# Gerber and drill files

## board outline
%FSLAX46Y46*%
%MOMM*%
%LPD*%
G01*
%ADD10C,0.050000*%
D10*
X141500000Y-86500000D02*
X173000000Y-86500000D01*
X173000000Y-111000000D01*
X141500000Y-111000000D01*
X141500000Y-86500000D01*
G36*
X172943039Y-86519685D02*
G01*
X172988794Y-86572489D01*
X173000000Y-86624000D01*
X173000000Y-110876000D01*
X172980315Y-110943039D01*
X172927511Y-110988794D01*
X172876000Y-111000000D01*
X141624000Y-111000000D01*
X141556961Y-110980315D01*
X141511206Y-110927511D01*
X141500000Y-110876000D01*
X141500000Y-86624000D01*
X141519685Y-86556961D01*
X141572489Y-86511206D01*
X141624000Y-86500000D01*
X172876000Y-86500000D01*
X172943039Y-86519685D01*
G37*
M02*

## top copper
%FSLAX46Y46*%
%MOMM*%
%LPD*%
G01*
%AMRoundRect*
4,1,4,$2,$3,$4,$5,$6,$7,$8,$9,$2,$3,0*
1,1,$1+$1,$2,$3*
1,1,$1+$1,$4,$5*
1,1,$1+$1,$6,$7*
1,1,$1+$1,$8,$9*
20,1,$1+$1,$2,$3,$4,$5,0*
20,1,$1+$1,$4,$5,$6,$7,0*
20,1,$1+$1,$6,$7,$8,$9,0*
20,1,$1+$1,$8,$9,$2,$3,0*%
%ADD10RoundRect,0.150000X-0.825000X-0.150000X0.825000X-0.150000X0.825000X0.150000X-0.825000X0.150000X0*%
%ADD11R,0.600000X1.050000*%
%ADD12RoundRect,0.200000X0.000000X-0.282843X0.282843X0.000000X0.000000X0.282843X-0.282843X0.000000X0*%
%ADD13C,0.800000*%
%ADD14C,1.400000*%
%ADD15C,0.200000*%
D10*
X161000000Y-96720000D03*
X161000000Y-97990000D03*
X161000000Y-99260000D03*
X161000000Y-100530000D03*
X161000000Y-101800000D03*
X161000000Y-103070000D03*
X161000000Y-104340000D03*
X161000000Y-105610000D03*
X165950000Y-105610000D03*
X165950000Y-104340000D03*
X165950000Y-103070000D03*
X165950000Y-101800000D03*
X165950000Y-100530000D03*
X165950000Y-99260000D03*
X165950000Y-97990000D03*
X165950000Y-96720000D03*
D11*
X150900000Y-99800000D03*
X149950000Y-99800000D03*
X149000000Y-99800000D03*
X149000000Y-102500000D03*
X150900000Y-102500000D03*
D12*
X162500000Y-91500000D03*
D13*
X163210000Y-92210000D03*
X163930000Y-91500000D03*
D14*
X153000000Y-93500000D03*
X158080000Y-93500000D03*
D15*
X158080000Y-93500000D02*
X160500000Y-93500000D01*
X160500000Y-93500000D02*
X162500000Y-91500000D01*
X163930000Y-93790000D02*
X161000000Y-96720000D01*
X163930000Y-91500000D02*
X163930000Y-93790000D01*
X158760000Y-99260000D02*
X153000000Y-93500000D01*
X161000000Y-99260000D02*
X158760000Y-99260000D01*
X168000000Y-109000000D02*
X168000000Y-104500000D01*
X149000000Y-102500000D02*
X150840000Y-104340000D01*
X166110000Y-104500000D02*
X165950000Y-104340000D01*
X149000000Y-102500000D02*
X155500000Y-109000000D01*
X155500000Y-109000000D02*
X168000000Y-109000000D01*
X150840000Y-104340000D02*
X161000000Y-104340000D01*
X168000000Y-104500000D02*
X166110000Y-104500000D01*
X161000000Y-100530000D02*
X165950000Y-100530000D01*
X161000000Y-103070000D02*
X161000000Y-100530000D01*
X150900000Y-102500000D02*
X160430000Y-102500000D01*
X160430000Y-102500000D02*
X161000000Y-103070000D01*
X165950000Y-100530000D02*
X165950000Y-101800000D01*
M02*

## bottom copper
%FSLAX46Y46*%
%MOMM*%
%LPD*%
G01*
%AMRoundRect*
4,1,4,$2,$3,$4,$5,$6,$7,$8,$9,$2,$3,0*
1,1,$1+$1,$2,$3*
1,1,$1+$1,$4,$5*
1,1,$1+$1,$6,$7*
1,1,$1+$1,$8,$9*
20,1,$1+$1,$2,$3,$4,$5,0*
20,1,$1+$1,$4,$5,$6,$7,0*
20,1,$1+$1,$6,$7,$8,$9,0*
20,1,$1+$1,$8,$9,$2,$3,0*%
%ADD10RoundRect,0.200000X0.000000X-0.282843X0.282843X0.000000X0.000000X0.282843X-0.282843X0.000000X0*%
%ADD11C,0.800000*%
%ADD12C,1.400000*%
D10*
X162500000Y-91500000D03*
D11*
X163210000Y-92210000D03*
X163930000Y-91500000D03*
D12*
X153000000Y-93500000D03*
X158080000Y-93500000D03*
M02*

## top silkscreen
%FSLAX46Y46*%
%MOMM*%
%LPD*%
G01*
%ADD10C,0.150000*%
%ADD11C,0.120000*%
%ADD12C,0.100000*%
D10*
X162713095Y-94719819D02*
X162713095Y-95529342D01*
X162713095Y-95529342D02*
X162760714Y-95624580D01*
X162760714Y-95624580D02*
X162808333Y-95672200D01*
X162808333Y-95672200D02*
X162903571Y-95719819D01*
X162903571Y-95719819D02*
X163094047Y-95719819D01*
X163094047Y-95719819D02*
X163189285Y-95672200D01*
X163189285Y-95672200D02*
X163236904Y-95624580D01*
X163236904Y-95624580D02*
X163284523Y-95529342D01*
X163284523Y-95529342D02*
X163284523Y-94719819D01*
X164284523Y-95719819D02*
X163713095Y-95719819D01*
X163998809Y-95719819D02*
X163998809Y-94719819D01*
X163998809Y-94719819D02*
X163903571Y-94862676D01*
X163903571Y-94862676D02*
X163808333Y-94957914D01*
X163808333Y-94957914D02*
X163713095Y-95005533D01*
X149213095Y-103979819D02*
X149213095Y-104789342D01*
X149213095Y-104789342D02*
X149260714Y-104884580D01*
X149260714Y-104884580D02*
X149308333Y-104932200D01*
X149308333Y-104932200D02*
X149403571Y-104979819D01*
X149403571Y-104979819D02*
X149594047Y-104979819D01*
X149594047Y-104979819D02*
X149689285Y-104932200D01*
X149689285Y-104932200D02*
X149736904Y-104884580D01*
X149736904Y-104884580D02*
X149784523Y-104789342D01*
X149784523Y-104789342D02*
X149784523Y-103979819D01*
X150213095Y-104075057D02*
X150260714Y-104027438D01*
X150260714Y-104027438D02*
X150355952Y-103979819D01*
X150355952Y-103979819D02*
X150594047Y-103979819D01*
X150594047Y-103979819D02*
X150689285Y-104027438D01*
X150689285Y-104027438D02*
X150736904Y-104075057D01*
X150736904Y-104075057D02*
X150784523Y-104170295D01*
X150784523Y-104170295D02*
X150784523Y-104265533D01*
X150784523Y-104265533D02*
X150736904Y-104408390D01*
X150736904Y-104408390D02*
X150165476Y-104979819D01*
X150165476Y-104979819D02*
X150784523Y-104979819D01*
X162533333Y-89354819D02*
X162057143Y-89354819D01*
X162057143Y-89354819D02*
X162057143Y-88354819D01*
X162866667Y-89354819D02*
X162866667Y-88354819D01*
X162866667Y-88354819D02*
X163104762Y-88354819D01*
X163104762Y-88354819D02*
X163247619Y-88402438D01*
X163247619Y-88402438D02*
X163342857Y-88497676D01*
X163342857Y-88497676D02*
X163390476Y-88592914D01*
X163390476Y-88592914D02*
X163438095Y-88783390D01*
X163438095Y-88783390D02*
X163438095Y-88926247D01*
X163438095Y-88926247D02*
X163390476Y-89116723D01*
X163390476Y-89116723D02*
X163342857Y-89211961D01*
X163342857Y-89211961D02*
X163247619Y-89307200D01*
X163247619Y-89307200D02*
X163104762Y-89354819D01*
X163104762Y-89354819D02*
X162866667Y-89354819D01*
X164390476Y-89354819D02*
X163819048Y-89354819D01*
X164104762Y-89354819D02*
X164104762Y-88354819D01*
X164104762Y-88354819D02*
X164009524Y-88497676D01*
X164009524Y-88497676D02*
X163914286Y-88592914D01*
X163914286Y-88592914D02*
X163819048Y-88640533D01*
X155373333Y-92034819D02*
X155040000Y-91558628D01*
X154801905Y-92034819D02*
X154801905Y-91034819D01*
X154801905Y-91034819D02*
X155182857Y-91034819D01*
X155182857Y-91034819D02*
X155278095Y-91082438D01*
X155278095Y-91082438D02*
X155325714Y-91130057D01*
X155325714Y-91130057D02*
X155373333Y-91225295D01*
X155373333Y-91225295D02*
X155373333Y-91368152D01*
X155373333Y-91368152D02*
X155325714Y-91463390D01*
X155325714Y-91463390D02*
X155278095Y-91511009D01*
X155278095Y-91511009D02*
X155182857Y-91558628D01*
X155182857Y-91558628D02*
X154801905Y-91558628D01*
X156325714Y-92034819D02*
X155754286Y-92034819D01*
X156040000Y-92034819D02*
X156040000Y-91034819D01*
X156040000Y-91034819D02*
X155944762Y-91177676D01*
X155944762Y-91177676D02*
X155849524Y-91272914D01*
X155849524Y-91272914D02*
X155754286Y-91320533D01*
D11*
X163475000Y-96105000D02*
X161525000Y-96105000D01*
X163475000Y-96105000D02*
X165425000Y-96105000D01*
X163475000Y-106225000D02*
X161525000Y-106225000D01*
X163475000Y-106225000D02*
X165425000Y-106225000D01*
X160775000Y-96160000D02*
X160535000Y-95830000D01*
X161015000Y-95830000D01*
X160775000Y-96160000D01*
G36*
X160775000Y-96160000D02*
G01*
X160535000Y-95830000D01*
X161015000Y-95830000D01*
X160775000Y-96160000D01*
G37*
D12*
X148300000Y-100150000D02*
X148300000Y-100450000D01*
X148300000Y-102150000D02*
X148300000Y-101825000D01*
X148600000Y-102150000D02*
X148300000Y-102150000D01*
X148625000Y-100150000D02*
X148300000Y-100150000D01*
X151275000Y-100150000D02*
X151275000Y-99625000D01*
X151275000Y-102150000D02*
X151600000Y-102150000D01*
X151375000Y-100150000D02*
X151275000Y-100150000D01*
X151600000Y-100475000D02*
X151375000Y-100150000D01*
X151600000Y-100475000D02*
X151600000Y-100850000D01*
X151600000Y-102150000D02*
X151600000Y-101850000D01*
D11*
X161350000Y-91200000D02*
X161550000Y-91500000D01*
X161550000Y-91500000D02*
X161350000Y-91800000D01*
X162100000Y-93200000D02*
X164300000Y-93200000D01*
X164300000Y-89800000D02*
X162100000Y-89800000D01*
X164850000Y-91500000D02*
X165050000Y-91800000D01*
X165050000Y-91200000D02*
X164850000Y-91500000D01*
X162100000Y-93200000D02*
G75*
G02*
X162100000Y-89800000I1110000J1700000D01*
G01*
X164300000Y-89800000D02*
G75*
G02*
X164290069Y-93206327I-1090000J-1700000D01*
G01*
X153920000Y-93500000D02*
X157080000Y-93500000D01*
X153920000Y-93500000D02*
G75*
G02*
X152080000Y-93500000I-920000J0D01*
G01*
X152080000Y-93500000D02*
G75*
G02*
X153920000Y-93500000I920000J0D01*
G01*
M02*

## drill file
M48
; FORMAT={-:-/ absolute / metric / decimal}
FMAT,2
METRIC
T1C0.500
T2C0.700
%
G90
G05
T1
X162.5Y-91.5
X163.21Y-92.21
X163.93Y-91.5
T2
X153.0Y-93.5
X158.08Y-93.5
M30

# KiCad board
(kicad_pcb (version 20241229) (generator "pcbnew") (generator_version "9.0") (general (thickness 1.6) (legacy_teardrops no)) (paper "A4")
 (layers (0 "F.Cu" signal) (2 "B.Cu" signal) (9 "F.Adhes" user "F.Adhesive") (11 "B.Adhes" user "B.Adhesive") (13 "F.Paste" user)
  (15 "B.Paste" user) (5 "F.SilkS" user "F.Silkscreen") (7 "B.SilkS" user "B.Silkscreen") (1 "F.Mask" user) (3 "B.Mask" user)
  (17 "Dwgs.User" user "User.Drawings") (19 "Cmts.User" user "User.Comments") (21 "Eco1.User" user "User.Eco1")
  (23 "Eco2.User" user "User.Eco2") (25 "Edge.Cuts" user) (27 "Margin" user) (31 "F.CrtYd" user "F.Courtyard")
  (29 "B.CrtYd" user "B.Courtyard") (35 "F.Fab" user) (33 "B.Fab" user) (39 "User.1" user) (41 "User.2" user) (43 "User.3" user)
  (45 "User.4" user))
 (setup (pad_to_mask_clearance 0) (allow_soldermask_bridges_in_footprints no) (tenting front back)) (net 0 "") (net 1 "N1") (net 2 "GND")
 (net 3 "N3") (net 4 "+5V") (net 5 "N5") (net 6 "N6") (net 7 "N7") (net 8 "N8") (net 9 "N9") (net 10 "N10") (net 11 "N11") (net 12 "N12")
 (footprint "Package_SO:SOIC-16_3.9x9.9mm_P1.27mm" (layer "F.Cu") (at 163.475 101.165)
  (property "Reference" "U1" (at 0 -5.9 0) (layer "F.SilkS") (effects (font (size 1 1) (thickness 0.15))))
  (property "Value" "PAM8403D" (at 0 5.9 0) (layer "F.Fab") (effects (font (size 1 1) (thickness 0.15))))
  (fp_line (start 0 -5.06) (end -1.95 -5.06) (stroke (width 0.12) (type solid)) (layer "F.SilkS"))
  (fp_line (start 0 -5.06) (end 1.95 -5.06) (stroke (width 0.12) (type solid)) (layer "F.SilkS"))
  (fp_line (start 0 5.06) (end -1.95 5.06) (stroke (width 0.12) (type solid)) (layer "F.SilkS"))
  (fp_line (start 0 5.06) (end 1.95 5.06) (stroke (width 0.12) (type solid)) (layer "F.SilkS"))
  (fp_poly (pts (xy -2.7 -5.005) (xy -2.94 -5.335) (xy -2.46 -5.335)) (stroke (width 0.12) (type solid)) (fill yes) (layer "F.SilkS"))
  (pad "1" smd roundrect (at -2.475 -4.445) (size 1.95 0.6) (layers "F.Cu" "F.Mask" "F.Paste") (roundrect_rratio 0.25) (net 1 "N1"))
  (pad "2" smd roundrect (at -2.475 -3.175) (size 1.95 0.6) (layers "F.Cu" "F.Mask" "F.Paste") (roundrect_rratio 0.25) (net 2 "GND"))
  (pad "3" smd roundrect (at -2.475 -1.905) (size 1.95 0.6) (layers "F.Cu" "F.Mask" "F.Paste") (roundrect_rratio 0.25) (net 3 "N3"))
  (pad "4" smd roundrect (at -2.475 -0.635) (size 1.95 0.6) (layers "F.Cu" "F.Mask" "F.Paste") (roundrect_rratio 0.25) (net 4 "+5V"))
  (pad "5" smd roundrect (at -2.475 0.635) (size 1.95 0.6) (layers "F.Cu" "F.Mask" "F.Paste") (roundrect_rratio 0.25) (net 4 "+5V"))
  (pad "6" smd roundrect (at -2.475 1.905) (size 1.95 0.6) (layers "F.Cu" "F.Mask" "F.Paste") (roundrect_rratio 0.25) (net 4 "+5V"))
  (pad "7" smd roundrect (at -2.475 3.175) (size 1.95 0.6) (layers "F.Cu" "F.Mask" "F.Paste") (roundrect_rratio 0.25) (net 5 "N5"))
  (pad "8" smd roundrect (at -2.475 4.445) (size 1.95 0.6) (layers "F.Cu" "F.Mask" "F.Paste") (roundrect_rratio 0.25) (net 2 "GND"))
  (pad "9" smd roundrect (at 2.475 4.445) (size 1.95 0.6) (layers "F.Cu" "F.Mask" "F.Paste") (roundrect_rratio 0.25) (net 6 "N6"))
  (pad "10" smd roundrect (at 2.475 3.175) (size 1.95 0.6) (layers "F.Cu" "F.Mask" "F.Paste") (roundrect_rratio 0.25) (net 5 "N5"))
  (pad "11" smd roundrect (at 2.475 1.905) (size 1.95 0.6) (layers "F.Cu" "F.Mask" "F.Paste") (roundrect_rratio 0.25) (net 2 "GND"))
  (pad "12" smd roundrect (at 2.475 0.635) (size 1.95 0.6) (layers "F.Cu" "F.Mask" "F.Paste") (roundrect_rratio 0.25) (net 4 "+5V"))
  (pad "13" smd roundrect (at 2.475 -0.635) (size 1.95 0.6) (layers "F.Cu" "F.Mask" "F.Paste") (roundrect_rratio 0.25) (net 4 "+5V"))
  (pad "14" smd roundrect (at 2.475 -1.905) (size 1.95 0.6) (layers "F.Cu" "F.Mask" "F.Paste") (roundrect_rratio 0.25) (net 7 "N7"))
  (pad "15" smd roundrect (at 2.475 -3.175) (size 1.95 0.6) (layers "F.Cu" "F.Mask" "F.Paste") (roundrect_rratio 0.25) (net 2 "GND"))
  (pad "16" smd roundrect (at 2.475 -4.445) (size 1.95 0.6) (layers "F.Cu" "F.Mask" "F.Paste") (roundrect_rratio 0.25) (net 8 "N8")))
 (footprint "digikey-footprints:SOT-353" (layer "F.Cu") (at 149.95 101.15 180)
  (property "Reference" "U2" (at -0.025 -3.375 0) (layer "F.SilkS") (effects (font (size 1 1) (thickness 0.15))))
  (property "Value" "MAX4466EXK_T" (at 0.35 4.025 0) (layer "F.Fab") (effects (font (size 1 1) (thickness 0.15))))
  (fp_line (start 1.65 1) (end 1.65 0.7) (stroke (width 0.1) (type solid)) (layer "F.SilkS"))
  (fp_line (start 1.65 -1) (end 1.65 -0.675) (stroke (width 0.1) (type solid)) (layer "F.SilkS"))
  (fp_line (start 1.35 -1) (end 1.65 -1) (stroke (width 0.1) (type solid)) (layer "F.SilkS"))
  (fp_line (start 1.325 1) (end 1.65 1) (stroke (width 0.1) (type solid)) (layer "F.SilkS"))
  (fp_line (start -1.325 1) (end -1.325 1.525) (stroke (width 0.1) (type solid)) (layer "F.SilkS"))
  (fp_line (start -1.325 -1) (end -1.65 -1) (stroke (width 0.1) (type solid)) (layer "F.SilkS"))
  (fp_line (start -1.425 1) (end -1.325 1) (stroke (width 0.1) (type solid)) (layer "F.SilkS"))
  (fp_line (start -1.65 0.675) (end -1.425 1) (stroke (width 0.1) (type solid)) (layer "F.SilkS"))
  (fp_line (start -1.65 0.675) (end -1.65 0.3) (stroke (width 0.1) (type solid)) (layer "F.SilkS"))
  (fp_line (start -1.65 -1) (end -1.65 -0.7) (stroke (width 0.1) (type solid)) (layer "F.SilkS"))
  (pad "1" smd rect (at -0.95 1.35 180) (size 0.6 1.05) (layers "F.Cu" "F.Mask" "F.Paste") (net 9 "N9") (solder_mask_margin 0.07))
  (pad "2" smd rect (at 0 1.35 180) (size 0.6 1.05) (layers "F.Cu" "F.Mask" "F.Paste") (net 2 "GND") (solder_mask_margin 0.07))
  (pad "3" smd rect (at 0.95 1.35 180) (size 0.6 1.05) (layers "F.Cu" "F.Mask" "F.Paste") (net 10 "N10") (solder_mask_margin 0.07))
  (pad "4" smd rect (at 0.95 -1.35 180) (size 0.6 1.05) (layers "F.Cu" "F.Mask" "F.Paste") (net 5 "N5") (solder_mask_margin 0.07))
  (pad "5" smd rect (at -0.95 -1.35 180) (size 0.6 1.05) (layers "F.Cu" "F.Mask" "F.Paste") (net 4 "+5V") (solder_mask_margin 0.07)))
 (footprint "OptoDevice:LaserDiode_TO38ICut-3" (layer "F.Cu") (at 162.5 91.5)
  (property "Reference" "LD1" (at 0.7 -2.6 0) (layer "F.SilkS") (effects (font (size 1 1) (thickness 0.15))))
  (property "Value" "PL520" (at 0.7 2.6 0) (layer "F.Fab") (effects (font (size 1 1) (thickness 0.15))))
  (fp_line (start -1.15 -0.3) (end -0.95 0) (stroke (width 0.12) (type solid)) (layer "F.SilkS"))
  (fp_line (start -0.95 0) (end -1.15 0.3) (stroke (width 0.12) (type solid)) (layer "F.SilkS"))
  (fp_line (start -0.4 1.7) (end 1.8 1.7) (stroke (width 0.12) (type solid)) (layer "F.SilkS"))
  (fp_line (start 1.8 -1.7) (end -0.4 -1.7) (stroke (width 0.12) (type solid)) (layer "F.SilkS"))
  (fp_line (start 2.35 0) (end 2.55 0.3) (stroke (width 0.12) (type solid)) (layer "F.SilkS"))
  (fp_line (start 2.55 -0.3) (end 2.35 0) (stroke (width 0.12) (type solid)) (layer "F.SilkS"))
  (fp_arc (start -0.4 1.7) (mid -1.320296 0) (end -0.4 -1.7) (stroke (width 0.12) (type solid)) (layer "F.SilkS"))
  (fp_arc (start 1.8 -1.7) (mid 2.729422 0.005888) (end 1.790069 1.706327) (stroke (width 0.12) (type solid)) (layer "F.SilkS"))
  (pad "1" thru_hole roundrect (at 0 0 45) (size 0.8 0.8) (drill 0.5) (layers "*.Cu" "*.Mask") (remove_unused_layers no)
   (roundrect_rratio 0.25) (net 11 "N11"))
  (pad "2" thru_hole circle (at 0.71 0.71) (size 0.8 0.8) (drill 0.5) (layers "*.Cu" "*.Mask") (remove_unused_layers no) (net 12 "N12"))
  (pad "3" thru_hole circle (at 1.43 0) (size 0.8 0.8) (drill 0.5) (layers "*.Cu" "*.Mask") (remove_unused_layers no) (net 1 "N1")))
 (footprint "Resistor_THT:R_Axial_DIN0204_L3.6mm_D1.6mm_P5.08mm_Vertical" (layer "F.Cu") (at 153 93.5)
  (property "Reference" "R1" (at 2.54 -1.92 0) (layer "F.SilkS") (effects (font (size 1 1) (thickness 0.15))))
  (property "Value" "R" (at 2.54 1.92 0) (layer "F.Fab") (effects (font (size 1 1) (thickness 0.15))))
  (fp_line (start 0.92 0) (end 4.08 0) (stroke (width 0.12) (type solid)) (layer "F.SilkS"))
  (fp_circle (center 0 0) (end 0.92 0) (stroke (width 0.12) (type solid)) (fill no) (layer "F.SilkS"))
  (pad "1" thru_hole circle (at 0 0) (size 1.4 1.4) (drill 0.7) (layers "*.Cu" "*.Mask") (remove_unused_layers no) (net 3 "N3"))
  (pad "2" thru_hole circle (at 5.08 0) (size 1.4 1.4) (drill 0.7) (layers "*.Cu" "*.Mask") (remove_unused_layers no) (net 11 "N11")))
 (gr_rect (start 141.5 86.5) (end 173 111) (stroke (width 0.05) (type default)) (fill no) (layer "Edge.Cuts"))
 (segment (start 158.08 93.5) (end 160.5 93.5) (width 0.2) (layer "F.Cu") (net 11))
 (segment (start 160.5 93.5) (end 162.5 91.5) (width 0.2) (layer "F.Cu") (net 11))
 (segment (start 163.93 93.79) (end 161 96.72) (width 0.2) (layer "F.Cu") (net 1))
 (segment (start 163.93 91.5) (end 163.93 93.79) (width 0.2) (layer "F.Cu") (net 1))
 (segment (start 158.76 99.26) (end 153 93.5) (width 0.2) (layer "F.Cu") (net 3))
 (segment (start 161 99.26) (end 158.76 99.26) (width 0.2) (layer "F.Cu") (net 3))
 (segment (start 168 109) (end 168 104.5) (width 0.2) (layer "F.Cu") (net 5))
 (segment (start 149 102.5) (end 150.84 104.34) (width 0.2) (layer "F.Cu") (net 5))
 (segment (start 166.11 104.5) (end 165.95 104.34) (width 0.2) (layer "F.Cu") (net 5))
 (segment (start 149 102.5) (end 155.5 109) (width 0.2) (layer "F.Cu") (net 5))
 (segment (start 155.5 109) (end 168 109) (width 0.2) (layer "F.Cu") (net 5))
 (segment (start 150.84 104.34) (end 161 104.34) (width 0.2) (layer "F.Cu") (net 5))
 (segment (start 168 104.5) (end 166.11 104.5) (width 0.2) (layer "F.Cu") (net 5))
 (segment (start 161 100.53) (end 165.95 100.53) (width 0.2) (layer "F.Cu") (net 4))
 (segment (start 161 103.07) (end 161 100.53) (width 0.2) (layer "F.Cu") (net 4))
 (segment (start 150.9 102.5) (end 160.43 102.5) (width 0.2) (layer "F.Cu") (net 4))
 (segment (start 160.43 102.5) (end 161 103.07) (width 0.2) (layer "F.Cu") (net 4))
 (segment (start 165.95 100.53) (end 165.95 101.8) (width 0.2) (layer "F.Cu") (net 4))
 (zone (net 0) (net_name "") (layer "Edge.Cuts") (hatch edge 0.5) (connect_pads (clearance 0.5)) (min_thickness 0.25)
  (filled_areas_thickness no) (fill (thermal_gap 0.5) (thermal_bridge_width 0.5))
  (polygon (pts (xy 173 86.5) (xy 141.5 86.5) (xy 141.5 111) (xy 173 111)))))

